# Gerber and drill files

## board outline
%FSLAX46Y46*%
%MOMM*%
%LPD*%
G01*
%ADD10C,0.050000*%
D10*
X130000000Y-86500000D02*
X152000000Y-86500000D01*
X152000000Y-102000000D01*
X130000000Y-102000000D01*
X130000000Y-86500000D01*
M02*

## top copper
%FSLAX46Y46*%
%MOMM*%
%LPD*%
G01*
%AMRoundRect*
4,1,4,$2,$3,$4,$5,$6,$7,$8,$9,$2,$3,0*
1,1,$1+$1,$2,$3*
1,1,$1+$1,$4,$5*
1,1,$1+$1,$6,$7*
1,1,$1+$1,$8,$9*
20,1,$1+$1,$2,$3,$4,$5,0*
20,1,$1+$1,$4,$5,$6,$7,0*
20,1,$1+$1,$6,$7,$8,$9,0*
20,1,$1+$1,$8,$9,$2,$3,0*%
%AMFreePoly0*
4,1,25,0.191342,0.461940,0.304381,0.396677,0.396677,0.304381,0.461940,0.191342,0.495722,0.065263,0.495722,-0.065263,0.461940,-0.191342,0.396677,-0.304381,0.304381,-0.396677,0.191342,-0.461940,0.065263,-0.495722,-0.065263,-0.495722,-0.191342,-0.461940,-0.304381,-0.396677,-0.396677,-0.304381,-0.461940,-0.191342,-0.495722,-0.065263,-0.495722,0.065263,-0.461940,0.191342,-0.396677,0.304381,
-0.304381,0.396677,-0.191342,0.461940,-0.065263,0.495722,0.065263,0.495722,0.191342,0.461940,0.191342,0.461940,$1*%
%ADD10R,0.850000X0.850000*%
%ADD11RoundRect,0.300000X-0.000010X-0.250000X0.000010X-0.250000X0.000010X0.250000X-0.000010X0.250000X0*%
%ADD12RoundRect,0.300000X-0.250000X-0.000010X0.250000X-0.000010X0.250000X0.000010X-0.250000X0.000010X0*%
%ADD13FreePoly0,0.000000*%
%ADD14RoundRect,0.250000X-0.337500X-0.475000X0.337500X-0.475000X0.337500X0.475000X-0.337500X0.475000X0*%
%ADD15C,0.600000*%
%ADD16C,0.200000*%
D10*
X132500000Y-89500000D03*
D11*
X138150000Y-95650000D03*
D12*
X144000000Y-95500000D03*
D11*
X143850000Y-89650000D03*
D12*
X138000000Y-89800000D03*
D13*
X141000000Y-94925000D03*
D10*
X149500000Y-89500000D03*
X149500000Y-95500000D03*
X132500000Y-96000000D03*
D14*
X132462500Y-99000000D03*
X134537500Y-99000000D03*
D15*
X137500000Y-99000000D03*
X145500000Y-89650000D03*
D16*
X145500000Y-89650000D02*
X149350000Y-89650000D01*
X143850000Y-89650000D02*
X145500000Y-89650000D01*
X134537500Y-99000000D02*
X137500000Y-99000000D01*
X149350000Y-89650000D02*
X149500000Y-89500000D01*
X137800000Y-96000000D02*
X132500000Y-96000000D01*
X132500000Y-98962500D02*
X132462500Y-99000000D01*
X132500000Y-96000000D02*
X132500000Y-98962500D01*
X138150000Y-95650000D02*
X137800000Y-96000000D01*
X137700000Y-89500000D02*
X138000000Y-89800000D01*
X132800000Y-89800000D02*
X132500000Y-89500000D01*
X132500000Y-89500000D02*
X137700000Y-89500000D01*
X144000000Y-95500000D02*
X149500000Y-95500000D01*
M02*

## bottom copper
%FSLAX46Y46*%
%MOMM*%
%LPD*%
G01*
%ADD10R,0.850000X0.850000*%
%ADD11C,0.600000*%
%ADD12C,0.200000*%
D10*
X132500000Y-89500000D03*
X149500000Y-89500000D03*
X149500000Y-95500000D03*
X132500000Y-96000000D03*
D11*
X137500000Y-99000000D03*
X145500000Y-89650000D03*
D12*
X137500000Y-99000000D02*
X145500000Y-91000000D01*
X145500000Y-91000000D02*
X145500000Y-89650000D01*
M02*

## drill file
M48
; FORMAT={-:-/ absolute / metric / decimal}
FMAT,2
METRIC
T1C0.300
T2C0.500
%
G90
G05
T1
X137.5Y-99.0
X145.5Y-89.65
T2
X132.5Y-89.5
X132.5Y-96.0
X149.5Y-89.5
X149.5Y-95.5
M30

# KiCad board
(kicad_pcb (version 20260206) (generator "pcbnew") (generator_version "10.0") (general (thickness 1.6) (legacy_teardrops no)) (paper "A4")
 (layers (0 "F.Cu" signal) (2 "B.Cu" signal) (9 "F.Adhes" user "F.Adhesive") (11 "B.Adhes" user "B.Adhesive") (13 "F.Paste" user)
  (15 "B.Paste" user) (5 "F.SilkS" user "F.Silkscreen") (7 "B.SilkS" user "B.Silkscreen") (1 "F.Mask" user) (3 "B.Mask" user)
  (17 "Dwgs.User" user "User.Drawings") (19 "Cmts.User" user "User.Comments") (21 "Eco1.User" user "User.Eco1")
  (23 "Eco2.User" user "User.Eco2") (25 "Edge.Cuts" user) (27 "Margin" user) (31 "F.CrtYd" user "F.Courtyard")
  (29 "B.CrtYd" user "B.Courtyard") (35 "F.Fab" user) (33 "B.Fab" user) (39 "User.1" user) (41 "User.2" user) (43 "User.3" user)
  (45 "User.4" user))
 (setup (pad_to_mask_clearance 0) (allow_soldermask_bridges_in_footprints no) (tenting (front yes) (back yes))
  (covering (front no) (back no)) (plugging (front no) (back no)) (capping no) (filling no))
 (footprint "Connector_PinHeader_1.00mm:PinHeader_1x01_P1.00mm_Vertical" (layer "F.Cu") (at 132.5 89.5)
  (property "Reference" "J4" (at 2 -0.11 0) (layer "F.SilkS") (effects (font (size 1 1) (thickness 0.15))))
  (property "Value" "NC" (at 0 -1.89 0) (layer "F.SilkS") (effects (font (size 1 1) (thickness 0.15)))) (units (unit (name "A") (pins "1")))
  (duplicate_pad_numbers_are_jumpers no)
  (pad "1" thru_hole rect (at 0 0) (size 0.85 0.85) (drill 0.5) (layers "*.Cu" "*.Mask") (remove_unused_layers no) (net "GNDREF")))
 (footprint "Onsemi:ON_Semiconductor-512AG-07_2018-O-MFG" (layer "F.Cu") (at 141 92.65)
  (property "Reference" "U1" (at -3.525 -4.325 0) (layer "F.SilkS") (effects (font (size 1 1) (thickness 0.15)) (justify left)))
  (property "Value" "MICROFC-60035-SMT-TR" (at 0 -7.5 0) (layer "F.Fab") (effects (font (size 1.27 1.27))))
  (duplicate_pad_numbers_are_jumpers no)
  (pad "1" smd roundrect (at -2.85 3) (size 0.6 1.1) (layers "F.Cu" "F.Mask" "F.Paste") (roundrect_rratio 0.5) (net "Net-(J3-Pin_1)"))
  (pad "2" smd roundrect (at 3 2.85) (size 1.1 0.6) (layers "F.Cu" "F.Mask" "F.Paste") (roundrect_rratio 0.5) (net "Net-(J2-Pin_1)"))
  (pad "3" smd roundrect (at 2.85 -3) (size 0.6 1.1) (layers "F.Cu" "F.Mask" "F.Paste") (roundrect_rratio 0.5) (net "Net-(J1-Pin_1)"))
  (pad "4" smd roundrect (at -3 -2.85) (size 1.1 0.6) (layers "F.Cu" "F.Mask" "F.Paste") (roundrect_rratio 0.5) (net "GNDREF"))
  (pad "5" smd custom (at 0 2.275) (size 1 1) (layers "F.Cu" "F.Mask" "F.Paste") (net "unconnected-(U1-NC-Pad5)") (thermal_bridge_angle 90)
   (options (clearance outline) (anchor circle)) (primitives)))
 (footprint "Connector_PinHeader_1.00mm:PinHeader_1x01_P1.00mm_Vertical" (layer "F.Cu") (at 149.5 89.5)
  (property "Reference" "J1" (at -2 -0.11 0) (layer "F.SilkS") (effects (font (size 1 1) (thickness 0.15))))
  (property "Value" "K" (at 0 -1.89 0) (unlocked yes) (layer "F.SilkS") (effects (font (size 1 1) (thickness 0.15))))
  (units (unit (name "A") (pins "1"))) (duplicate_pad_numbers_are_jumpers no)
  (pad "1" thru_hole rect (at 0 0) (size 0.85 0.85) (drill 0.5) (layers "*.Cu" "*.Mask") (remove_unused_layers no) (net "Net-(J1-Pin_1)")))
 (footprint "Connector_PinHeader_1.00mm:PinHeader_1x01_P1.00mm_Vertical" (layer "F.Cu") (at 149.5 95.5)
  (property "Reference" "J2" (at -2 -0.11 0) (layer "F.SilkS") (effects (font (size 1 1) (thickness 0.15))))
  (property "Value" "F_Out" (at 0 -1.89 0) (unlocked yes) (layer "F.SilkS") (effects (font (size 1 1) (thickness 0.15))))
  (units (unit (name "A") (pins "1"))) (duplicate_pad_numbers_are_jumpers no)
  (pad "1" thru_hole rect (at 0 0) (size 0.85 0.85) (drill 0.5) (layers "*.Cu" "*.Mask") (remove_unused_layers no) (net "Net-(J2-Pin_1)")))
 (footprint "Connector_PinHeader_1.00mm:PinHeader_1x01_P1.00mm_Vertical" (layer "F.Cu") (at 132.5 96)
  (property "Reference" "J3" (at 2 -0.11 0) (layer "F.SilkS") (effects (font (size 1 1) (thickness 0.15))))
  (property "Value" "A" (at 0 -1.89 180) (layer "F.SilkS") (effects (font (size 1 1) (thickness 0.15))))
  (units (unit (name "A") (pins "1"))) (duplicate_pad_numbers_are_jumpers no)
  (pad "1" thru_hole rect (at 0 0) (size 0.85 0.85) (drill 0.5) (layers "*.Cu" "*.Mask") (remove_unused_layers no) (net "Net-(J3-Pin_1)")))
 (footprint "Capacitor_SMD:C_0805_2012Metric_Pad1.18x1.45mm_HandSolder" (layer "F.Cu") (at 133.5 99)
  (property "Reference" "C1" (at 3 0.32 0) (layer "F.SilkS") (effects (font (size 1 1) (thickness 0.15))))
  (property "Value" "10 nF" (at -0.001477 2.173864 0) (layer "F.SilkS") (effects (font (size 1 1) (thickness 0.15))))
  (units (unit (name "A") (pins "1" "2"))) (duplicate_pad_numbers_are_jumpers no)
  (pad "1" smd roundrect (at -1.0375 0) (size 1.175 1.45) (layers "F.Cu" "F.Mask" "F.Paste") (roundrect_rratio 0.212766)
   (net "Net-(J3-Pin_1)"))
  (pad "2" smd roundrect (at 1.0375 0) (size 1.175 1.45) (layers "F.Cu" "F.Mask" "F.Paste") (roundrect_rratio 0.212766)
   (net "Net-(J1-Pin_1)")))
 (gr_rect (start 130 86.5) (end 152 102) (stroke (width 0.05) (type default)) (fill no) (layer "Edge.Cuts"))
 (segment (start 145.5 89.65) (end 149.35 89.65) (width 0.2) (layer "F.Cu") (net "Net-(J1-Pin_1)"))
 (segment (start 143.85 89.65) (end 145.5 89.65) (width 0.2) (layer "F.Cu") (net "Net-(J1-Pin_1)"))
 (segment (start 134.5375 99) (end 137.5 99) (width 0.2) (layer "F.Cu") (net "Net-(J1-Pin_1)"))
 (segment (start 149.35 89.65) (end 149.5 89.5) (width 0.2) (layer "F.Cu") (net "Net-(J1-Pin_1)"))
 (via (at 137.5 99) (size 0.6) (drill 0.3) (layers "F.Cu" "B.Cu") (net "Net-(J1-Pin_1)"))
 (via (at 145.5 89.65) (size 0.6) (drill 0.3) (layers "F.Cu" "B.Cu") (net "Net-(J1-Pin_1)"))
 (segment (start 137.5 99) (end 145.5 91) (width 0.2) (layer "B.Cu") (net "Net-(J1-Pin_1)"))
 (segment (start 145.5 91) (end 145.5 89.65) (width 0.2) (layer "B.Cu") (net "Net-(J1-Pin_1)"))
 (segment (start 137.8 96) (end 132.5 96) (width 0.2) (layer "F.Cu") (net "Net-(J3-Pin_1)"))
 (segment (start 132.5 98.9625) (end 132.4625 99) (width 0.2) (layer "F.Cu") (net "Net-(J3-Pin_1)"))
 (segment (start 132.5 96) (end 132.5 98.9625) (width 0.2) (layer "F.Cu") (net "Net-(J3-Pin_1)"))
 (segment (start 138.15 95.65) (end 137.8 96) (width 0.2) (layer "F.Cu") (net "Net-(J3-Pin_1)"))
 (segment (start 137.7 89.5) (end 138 89.8) (width 0.2) (layer "F.Cu") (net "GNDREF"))
 (segment (start 132.8 89.8) (end 132.5 89.5) (width 0.2) (layer "F.Cu") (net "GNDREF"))
 (segment (start 132.5 89.5) (end 137.7 89.5) (width 0.2) (layer "F.Cu") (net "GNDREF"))
 (segment (start 144 95.5) (end 149.5 95.5) (width 0.2) (layer "F.Cu") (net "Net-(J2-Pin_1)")))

